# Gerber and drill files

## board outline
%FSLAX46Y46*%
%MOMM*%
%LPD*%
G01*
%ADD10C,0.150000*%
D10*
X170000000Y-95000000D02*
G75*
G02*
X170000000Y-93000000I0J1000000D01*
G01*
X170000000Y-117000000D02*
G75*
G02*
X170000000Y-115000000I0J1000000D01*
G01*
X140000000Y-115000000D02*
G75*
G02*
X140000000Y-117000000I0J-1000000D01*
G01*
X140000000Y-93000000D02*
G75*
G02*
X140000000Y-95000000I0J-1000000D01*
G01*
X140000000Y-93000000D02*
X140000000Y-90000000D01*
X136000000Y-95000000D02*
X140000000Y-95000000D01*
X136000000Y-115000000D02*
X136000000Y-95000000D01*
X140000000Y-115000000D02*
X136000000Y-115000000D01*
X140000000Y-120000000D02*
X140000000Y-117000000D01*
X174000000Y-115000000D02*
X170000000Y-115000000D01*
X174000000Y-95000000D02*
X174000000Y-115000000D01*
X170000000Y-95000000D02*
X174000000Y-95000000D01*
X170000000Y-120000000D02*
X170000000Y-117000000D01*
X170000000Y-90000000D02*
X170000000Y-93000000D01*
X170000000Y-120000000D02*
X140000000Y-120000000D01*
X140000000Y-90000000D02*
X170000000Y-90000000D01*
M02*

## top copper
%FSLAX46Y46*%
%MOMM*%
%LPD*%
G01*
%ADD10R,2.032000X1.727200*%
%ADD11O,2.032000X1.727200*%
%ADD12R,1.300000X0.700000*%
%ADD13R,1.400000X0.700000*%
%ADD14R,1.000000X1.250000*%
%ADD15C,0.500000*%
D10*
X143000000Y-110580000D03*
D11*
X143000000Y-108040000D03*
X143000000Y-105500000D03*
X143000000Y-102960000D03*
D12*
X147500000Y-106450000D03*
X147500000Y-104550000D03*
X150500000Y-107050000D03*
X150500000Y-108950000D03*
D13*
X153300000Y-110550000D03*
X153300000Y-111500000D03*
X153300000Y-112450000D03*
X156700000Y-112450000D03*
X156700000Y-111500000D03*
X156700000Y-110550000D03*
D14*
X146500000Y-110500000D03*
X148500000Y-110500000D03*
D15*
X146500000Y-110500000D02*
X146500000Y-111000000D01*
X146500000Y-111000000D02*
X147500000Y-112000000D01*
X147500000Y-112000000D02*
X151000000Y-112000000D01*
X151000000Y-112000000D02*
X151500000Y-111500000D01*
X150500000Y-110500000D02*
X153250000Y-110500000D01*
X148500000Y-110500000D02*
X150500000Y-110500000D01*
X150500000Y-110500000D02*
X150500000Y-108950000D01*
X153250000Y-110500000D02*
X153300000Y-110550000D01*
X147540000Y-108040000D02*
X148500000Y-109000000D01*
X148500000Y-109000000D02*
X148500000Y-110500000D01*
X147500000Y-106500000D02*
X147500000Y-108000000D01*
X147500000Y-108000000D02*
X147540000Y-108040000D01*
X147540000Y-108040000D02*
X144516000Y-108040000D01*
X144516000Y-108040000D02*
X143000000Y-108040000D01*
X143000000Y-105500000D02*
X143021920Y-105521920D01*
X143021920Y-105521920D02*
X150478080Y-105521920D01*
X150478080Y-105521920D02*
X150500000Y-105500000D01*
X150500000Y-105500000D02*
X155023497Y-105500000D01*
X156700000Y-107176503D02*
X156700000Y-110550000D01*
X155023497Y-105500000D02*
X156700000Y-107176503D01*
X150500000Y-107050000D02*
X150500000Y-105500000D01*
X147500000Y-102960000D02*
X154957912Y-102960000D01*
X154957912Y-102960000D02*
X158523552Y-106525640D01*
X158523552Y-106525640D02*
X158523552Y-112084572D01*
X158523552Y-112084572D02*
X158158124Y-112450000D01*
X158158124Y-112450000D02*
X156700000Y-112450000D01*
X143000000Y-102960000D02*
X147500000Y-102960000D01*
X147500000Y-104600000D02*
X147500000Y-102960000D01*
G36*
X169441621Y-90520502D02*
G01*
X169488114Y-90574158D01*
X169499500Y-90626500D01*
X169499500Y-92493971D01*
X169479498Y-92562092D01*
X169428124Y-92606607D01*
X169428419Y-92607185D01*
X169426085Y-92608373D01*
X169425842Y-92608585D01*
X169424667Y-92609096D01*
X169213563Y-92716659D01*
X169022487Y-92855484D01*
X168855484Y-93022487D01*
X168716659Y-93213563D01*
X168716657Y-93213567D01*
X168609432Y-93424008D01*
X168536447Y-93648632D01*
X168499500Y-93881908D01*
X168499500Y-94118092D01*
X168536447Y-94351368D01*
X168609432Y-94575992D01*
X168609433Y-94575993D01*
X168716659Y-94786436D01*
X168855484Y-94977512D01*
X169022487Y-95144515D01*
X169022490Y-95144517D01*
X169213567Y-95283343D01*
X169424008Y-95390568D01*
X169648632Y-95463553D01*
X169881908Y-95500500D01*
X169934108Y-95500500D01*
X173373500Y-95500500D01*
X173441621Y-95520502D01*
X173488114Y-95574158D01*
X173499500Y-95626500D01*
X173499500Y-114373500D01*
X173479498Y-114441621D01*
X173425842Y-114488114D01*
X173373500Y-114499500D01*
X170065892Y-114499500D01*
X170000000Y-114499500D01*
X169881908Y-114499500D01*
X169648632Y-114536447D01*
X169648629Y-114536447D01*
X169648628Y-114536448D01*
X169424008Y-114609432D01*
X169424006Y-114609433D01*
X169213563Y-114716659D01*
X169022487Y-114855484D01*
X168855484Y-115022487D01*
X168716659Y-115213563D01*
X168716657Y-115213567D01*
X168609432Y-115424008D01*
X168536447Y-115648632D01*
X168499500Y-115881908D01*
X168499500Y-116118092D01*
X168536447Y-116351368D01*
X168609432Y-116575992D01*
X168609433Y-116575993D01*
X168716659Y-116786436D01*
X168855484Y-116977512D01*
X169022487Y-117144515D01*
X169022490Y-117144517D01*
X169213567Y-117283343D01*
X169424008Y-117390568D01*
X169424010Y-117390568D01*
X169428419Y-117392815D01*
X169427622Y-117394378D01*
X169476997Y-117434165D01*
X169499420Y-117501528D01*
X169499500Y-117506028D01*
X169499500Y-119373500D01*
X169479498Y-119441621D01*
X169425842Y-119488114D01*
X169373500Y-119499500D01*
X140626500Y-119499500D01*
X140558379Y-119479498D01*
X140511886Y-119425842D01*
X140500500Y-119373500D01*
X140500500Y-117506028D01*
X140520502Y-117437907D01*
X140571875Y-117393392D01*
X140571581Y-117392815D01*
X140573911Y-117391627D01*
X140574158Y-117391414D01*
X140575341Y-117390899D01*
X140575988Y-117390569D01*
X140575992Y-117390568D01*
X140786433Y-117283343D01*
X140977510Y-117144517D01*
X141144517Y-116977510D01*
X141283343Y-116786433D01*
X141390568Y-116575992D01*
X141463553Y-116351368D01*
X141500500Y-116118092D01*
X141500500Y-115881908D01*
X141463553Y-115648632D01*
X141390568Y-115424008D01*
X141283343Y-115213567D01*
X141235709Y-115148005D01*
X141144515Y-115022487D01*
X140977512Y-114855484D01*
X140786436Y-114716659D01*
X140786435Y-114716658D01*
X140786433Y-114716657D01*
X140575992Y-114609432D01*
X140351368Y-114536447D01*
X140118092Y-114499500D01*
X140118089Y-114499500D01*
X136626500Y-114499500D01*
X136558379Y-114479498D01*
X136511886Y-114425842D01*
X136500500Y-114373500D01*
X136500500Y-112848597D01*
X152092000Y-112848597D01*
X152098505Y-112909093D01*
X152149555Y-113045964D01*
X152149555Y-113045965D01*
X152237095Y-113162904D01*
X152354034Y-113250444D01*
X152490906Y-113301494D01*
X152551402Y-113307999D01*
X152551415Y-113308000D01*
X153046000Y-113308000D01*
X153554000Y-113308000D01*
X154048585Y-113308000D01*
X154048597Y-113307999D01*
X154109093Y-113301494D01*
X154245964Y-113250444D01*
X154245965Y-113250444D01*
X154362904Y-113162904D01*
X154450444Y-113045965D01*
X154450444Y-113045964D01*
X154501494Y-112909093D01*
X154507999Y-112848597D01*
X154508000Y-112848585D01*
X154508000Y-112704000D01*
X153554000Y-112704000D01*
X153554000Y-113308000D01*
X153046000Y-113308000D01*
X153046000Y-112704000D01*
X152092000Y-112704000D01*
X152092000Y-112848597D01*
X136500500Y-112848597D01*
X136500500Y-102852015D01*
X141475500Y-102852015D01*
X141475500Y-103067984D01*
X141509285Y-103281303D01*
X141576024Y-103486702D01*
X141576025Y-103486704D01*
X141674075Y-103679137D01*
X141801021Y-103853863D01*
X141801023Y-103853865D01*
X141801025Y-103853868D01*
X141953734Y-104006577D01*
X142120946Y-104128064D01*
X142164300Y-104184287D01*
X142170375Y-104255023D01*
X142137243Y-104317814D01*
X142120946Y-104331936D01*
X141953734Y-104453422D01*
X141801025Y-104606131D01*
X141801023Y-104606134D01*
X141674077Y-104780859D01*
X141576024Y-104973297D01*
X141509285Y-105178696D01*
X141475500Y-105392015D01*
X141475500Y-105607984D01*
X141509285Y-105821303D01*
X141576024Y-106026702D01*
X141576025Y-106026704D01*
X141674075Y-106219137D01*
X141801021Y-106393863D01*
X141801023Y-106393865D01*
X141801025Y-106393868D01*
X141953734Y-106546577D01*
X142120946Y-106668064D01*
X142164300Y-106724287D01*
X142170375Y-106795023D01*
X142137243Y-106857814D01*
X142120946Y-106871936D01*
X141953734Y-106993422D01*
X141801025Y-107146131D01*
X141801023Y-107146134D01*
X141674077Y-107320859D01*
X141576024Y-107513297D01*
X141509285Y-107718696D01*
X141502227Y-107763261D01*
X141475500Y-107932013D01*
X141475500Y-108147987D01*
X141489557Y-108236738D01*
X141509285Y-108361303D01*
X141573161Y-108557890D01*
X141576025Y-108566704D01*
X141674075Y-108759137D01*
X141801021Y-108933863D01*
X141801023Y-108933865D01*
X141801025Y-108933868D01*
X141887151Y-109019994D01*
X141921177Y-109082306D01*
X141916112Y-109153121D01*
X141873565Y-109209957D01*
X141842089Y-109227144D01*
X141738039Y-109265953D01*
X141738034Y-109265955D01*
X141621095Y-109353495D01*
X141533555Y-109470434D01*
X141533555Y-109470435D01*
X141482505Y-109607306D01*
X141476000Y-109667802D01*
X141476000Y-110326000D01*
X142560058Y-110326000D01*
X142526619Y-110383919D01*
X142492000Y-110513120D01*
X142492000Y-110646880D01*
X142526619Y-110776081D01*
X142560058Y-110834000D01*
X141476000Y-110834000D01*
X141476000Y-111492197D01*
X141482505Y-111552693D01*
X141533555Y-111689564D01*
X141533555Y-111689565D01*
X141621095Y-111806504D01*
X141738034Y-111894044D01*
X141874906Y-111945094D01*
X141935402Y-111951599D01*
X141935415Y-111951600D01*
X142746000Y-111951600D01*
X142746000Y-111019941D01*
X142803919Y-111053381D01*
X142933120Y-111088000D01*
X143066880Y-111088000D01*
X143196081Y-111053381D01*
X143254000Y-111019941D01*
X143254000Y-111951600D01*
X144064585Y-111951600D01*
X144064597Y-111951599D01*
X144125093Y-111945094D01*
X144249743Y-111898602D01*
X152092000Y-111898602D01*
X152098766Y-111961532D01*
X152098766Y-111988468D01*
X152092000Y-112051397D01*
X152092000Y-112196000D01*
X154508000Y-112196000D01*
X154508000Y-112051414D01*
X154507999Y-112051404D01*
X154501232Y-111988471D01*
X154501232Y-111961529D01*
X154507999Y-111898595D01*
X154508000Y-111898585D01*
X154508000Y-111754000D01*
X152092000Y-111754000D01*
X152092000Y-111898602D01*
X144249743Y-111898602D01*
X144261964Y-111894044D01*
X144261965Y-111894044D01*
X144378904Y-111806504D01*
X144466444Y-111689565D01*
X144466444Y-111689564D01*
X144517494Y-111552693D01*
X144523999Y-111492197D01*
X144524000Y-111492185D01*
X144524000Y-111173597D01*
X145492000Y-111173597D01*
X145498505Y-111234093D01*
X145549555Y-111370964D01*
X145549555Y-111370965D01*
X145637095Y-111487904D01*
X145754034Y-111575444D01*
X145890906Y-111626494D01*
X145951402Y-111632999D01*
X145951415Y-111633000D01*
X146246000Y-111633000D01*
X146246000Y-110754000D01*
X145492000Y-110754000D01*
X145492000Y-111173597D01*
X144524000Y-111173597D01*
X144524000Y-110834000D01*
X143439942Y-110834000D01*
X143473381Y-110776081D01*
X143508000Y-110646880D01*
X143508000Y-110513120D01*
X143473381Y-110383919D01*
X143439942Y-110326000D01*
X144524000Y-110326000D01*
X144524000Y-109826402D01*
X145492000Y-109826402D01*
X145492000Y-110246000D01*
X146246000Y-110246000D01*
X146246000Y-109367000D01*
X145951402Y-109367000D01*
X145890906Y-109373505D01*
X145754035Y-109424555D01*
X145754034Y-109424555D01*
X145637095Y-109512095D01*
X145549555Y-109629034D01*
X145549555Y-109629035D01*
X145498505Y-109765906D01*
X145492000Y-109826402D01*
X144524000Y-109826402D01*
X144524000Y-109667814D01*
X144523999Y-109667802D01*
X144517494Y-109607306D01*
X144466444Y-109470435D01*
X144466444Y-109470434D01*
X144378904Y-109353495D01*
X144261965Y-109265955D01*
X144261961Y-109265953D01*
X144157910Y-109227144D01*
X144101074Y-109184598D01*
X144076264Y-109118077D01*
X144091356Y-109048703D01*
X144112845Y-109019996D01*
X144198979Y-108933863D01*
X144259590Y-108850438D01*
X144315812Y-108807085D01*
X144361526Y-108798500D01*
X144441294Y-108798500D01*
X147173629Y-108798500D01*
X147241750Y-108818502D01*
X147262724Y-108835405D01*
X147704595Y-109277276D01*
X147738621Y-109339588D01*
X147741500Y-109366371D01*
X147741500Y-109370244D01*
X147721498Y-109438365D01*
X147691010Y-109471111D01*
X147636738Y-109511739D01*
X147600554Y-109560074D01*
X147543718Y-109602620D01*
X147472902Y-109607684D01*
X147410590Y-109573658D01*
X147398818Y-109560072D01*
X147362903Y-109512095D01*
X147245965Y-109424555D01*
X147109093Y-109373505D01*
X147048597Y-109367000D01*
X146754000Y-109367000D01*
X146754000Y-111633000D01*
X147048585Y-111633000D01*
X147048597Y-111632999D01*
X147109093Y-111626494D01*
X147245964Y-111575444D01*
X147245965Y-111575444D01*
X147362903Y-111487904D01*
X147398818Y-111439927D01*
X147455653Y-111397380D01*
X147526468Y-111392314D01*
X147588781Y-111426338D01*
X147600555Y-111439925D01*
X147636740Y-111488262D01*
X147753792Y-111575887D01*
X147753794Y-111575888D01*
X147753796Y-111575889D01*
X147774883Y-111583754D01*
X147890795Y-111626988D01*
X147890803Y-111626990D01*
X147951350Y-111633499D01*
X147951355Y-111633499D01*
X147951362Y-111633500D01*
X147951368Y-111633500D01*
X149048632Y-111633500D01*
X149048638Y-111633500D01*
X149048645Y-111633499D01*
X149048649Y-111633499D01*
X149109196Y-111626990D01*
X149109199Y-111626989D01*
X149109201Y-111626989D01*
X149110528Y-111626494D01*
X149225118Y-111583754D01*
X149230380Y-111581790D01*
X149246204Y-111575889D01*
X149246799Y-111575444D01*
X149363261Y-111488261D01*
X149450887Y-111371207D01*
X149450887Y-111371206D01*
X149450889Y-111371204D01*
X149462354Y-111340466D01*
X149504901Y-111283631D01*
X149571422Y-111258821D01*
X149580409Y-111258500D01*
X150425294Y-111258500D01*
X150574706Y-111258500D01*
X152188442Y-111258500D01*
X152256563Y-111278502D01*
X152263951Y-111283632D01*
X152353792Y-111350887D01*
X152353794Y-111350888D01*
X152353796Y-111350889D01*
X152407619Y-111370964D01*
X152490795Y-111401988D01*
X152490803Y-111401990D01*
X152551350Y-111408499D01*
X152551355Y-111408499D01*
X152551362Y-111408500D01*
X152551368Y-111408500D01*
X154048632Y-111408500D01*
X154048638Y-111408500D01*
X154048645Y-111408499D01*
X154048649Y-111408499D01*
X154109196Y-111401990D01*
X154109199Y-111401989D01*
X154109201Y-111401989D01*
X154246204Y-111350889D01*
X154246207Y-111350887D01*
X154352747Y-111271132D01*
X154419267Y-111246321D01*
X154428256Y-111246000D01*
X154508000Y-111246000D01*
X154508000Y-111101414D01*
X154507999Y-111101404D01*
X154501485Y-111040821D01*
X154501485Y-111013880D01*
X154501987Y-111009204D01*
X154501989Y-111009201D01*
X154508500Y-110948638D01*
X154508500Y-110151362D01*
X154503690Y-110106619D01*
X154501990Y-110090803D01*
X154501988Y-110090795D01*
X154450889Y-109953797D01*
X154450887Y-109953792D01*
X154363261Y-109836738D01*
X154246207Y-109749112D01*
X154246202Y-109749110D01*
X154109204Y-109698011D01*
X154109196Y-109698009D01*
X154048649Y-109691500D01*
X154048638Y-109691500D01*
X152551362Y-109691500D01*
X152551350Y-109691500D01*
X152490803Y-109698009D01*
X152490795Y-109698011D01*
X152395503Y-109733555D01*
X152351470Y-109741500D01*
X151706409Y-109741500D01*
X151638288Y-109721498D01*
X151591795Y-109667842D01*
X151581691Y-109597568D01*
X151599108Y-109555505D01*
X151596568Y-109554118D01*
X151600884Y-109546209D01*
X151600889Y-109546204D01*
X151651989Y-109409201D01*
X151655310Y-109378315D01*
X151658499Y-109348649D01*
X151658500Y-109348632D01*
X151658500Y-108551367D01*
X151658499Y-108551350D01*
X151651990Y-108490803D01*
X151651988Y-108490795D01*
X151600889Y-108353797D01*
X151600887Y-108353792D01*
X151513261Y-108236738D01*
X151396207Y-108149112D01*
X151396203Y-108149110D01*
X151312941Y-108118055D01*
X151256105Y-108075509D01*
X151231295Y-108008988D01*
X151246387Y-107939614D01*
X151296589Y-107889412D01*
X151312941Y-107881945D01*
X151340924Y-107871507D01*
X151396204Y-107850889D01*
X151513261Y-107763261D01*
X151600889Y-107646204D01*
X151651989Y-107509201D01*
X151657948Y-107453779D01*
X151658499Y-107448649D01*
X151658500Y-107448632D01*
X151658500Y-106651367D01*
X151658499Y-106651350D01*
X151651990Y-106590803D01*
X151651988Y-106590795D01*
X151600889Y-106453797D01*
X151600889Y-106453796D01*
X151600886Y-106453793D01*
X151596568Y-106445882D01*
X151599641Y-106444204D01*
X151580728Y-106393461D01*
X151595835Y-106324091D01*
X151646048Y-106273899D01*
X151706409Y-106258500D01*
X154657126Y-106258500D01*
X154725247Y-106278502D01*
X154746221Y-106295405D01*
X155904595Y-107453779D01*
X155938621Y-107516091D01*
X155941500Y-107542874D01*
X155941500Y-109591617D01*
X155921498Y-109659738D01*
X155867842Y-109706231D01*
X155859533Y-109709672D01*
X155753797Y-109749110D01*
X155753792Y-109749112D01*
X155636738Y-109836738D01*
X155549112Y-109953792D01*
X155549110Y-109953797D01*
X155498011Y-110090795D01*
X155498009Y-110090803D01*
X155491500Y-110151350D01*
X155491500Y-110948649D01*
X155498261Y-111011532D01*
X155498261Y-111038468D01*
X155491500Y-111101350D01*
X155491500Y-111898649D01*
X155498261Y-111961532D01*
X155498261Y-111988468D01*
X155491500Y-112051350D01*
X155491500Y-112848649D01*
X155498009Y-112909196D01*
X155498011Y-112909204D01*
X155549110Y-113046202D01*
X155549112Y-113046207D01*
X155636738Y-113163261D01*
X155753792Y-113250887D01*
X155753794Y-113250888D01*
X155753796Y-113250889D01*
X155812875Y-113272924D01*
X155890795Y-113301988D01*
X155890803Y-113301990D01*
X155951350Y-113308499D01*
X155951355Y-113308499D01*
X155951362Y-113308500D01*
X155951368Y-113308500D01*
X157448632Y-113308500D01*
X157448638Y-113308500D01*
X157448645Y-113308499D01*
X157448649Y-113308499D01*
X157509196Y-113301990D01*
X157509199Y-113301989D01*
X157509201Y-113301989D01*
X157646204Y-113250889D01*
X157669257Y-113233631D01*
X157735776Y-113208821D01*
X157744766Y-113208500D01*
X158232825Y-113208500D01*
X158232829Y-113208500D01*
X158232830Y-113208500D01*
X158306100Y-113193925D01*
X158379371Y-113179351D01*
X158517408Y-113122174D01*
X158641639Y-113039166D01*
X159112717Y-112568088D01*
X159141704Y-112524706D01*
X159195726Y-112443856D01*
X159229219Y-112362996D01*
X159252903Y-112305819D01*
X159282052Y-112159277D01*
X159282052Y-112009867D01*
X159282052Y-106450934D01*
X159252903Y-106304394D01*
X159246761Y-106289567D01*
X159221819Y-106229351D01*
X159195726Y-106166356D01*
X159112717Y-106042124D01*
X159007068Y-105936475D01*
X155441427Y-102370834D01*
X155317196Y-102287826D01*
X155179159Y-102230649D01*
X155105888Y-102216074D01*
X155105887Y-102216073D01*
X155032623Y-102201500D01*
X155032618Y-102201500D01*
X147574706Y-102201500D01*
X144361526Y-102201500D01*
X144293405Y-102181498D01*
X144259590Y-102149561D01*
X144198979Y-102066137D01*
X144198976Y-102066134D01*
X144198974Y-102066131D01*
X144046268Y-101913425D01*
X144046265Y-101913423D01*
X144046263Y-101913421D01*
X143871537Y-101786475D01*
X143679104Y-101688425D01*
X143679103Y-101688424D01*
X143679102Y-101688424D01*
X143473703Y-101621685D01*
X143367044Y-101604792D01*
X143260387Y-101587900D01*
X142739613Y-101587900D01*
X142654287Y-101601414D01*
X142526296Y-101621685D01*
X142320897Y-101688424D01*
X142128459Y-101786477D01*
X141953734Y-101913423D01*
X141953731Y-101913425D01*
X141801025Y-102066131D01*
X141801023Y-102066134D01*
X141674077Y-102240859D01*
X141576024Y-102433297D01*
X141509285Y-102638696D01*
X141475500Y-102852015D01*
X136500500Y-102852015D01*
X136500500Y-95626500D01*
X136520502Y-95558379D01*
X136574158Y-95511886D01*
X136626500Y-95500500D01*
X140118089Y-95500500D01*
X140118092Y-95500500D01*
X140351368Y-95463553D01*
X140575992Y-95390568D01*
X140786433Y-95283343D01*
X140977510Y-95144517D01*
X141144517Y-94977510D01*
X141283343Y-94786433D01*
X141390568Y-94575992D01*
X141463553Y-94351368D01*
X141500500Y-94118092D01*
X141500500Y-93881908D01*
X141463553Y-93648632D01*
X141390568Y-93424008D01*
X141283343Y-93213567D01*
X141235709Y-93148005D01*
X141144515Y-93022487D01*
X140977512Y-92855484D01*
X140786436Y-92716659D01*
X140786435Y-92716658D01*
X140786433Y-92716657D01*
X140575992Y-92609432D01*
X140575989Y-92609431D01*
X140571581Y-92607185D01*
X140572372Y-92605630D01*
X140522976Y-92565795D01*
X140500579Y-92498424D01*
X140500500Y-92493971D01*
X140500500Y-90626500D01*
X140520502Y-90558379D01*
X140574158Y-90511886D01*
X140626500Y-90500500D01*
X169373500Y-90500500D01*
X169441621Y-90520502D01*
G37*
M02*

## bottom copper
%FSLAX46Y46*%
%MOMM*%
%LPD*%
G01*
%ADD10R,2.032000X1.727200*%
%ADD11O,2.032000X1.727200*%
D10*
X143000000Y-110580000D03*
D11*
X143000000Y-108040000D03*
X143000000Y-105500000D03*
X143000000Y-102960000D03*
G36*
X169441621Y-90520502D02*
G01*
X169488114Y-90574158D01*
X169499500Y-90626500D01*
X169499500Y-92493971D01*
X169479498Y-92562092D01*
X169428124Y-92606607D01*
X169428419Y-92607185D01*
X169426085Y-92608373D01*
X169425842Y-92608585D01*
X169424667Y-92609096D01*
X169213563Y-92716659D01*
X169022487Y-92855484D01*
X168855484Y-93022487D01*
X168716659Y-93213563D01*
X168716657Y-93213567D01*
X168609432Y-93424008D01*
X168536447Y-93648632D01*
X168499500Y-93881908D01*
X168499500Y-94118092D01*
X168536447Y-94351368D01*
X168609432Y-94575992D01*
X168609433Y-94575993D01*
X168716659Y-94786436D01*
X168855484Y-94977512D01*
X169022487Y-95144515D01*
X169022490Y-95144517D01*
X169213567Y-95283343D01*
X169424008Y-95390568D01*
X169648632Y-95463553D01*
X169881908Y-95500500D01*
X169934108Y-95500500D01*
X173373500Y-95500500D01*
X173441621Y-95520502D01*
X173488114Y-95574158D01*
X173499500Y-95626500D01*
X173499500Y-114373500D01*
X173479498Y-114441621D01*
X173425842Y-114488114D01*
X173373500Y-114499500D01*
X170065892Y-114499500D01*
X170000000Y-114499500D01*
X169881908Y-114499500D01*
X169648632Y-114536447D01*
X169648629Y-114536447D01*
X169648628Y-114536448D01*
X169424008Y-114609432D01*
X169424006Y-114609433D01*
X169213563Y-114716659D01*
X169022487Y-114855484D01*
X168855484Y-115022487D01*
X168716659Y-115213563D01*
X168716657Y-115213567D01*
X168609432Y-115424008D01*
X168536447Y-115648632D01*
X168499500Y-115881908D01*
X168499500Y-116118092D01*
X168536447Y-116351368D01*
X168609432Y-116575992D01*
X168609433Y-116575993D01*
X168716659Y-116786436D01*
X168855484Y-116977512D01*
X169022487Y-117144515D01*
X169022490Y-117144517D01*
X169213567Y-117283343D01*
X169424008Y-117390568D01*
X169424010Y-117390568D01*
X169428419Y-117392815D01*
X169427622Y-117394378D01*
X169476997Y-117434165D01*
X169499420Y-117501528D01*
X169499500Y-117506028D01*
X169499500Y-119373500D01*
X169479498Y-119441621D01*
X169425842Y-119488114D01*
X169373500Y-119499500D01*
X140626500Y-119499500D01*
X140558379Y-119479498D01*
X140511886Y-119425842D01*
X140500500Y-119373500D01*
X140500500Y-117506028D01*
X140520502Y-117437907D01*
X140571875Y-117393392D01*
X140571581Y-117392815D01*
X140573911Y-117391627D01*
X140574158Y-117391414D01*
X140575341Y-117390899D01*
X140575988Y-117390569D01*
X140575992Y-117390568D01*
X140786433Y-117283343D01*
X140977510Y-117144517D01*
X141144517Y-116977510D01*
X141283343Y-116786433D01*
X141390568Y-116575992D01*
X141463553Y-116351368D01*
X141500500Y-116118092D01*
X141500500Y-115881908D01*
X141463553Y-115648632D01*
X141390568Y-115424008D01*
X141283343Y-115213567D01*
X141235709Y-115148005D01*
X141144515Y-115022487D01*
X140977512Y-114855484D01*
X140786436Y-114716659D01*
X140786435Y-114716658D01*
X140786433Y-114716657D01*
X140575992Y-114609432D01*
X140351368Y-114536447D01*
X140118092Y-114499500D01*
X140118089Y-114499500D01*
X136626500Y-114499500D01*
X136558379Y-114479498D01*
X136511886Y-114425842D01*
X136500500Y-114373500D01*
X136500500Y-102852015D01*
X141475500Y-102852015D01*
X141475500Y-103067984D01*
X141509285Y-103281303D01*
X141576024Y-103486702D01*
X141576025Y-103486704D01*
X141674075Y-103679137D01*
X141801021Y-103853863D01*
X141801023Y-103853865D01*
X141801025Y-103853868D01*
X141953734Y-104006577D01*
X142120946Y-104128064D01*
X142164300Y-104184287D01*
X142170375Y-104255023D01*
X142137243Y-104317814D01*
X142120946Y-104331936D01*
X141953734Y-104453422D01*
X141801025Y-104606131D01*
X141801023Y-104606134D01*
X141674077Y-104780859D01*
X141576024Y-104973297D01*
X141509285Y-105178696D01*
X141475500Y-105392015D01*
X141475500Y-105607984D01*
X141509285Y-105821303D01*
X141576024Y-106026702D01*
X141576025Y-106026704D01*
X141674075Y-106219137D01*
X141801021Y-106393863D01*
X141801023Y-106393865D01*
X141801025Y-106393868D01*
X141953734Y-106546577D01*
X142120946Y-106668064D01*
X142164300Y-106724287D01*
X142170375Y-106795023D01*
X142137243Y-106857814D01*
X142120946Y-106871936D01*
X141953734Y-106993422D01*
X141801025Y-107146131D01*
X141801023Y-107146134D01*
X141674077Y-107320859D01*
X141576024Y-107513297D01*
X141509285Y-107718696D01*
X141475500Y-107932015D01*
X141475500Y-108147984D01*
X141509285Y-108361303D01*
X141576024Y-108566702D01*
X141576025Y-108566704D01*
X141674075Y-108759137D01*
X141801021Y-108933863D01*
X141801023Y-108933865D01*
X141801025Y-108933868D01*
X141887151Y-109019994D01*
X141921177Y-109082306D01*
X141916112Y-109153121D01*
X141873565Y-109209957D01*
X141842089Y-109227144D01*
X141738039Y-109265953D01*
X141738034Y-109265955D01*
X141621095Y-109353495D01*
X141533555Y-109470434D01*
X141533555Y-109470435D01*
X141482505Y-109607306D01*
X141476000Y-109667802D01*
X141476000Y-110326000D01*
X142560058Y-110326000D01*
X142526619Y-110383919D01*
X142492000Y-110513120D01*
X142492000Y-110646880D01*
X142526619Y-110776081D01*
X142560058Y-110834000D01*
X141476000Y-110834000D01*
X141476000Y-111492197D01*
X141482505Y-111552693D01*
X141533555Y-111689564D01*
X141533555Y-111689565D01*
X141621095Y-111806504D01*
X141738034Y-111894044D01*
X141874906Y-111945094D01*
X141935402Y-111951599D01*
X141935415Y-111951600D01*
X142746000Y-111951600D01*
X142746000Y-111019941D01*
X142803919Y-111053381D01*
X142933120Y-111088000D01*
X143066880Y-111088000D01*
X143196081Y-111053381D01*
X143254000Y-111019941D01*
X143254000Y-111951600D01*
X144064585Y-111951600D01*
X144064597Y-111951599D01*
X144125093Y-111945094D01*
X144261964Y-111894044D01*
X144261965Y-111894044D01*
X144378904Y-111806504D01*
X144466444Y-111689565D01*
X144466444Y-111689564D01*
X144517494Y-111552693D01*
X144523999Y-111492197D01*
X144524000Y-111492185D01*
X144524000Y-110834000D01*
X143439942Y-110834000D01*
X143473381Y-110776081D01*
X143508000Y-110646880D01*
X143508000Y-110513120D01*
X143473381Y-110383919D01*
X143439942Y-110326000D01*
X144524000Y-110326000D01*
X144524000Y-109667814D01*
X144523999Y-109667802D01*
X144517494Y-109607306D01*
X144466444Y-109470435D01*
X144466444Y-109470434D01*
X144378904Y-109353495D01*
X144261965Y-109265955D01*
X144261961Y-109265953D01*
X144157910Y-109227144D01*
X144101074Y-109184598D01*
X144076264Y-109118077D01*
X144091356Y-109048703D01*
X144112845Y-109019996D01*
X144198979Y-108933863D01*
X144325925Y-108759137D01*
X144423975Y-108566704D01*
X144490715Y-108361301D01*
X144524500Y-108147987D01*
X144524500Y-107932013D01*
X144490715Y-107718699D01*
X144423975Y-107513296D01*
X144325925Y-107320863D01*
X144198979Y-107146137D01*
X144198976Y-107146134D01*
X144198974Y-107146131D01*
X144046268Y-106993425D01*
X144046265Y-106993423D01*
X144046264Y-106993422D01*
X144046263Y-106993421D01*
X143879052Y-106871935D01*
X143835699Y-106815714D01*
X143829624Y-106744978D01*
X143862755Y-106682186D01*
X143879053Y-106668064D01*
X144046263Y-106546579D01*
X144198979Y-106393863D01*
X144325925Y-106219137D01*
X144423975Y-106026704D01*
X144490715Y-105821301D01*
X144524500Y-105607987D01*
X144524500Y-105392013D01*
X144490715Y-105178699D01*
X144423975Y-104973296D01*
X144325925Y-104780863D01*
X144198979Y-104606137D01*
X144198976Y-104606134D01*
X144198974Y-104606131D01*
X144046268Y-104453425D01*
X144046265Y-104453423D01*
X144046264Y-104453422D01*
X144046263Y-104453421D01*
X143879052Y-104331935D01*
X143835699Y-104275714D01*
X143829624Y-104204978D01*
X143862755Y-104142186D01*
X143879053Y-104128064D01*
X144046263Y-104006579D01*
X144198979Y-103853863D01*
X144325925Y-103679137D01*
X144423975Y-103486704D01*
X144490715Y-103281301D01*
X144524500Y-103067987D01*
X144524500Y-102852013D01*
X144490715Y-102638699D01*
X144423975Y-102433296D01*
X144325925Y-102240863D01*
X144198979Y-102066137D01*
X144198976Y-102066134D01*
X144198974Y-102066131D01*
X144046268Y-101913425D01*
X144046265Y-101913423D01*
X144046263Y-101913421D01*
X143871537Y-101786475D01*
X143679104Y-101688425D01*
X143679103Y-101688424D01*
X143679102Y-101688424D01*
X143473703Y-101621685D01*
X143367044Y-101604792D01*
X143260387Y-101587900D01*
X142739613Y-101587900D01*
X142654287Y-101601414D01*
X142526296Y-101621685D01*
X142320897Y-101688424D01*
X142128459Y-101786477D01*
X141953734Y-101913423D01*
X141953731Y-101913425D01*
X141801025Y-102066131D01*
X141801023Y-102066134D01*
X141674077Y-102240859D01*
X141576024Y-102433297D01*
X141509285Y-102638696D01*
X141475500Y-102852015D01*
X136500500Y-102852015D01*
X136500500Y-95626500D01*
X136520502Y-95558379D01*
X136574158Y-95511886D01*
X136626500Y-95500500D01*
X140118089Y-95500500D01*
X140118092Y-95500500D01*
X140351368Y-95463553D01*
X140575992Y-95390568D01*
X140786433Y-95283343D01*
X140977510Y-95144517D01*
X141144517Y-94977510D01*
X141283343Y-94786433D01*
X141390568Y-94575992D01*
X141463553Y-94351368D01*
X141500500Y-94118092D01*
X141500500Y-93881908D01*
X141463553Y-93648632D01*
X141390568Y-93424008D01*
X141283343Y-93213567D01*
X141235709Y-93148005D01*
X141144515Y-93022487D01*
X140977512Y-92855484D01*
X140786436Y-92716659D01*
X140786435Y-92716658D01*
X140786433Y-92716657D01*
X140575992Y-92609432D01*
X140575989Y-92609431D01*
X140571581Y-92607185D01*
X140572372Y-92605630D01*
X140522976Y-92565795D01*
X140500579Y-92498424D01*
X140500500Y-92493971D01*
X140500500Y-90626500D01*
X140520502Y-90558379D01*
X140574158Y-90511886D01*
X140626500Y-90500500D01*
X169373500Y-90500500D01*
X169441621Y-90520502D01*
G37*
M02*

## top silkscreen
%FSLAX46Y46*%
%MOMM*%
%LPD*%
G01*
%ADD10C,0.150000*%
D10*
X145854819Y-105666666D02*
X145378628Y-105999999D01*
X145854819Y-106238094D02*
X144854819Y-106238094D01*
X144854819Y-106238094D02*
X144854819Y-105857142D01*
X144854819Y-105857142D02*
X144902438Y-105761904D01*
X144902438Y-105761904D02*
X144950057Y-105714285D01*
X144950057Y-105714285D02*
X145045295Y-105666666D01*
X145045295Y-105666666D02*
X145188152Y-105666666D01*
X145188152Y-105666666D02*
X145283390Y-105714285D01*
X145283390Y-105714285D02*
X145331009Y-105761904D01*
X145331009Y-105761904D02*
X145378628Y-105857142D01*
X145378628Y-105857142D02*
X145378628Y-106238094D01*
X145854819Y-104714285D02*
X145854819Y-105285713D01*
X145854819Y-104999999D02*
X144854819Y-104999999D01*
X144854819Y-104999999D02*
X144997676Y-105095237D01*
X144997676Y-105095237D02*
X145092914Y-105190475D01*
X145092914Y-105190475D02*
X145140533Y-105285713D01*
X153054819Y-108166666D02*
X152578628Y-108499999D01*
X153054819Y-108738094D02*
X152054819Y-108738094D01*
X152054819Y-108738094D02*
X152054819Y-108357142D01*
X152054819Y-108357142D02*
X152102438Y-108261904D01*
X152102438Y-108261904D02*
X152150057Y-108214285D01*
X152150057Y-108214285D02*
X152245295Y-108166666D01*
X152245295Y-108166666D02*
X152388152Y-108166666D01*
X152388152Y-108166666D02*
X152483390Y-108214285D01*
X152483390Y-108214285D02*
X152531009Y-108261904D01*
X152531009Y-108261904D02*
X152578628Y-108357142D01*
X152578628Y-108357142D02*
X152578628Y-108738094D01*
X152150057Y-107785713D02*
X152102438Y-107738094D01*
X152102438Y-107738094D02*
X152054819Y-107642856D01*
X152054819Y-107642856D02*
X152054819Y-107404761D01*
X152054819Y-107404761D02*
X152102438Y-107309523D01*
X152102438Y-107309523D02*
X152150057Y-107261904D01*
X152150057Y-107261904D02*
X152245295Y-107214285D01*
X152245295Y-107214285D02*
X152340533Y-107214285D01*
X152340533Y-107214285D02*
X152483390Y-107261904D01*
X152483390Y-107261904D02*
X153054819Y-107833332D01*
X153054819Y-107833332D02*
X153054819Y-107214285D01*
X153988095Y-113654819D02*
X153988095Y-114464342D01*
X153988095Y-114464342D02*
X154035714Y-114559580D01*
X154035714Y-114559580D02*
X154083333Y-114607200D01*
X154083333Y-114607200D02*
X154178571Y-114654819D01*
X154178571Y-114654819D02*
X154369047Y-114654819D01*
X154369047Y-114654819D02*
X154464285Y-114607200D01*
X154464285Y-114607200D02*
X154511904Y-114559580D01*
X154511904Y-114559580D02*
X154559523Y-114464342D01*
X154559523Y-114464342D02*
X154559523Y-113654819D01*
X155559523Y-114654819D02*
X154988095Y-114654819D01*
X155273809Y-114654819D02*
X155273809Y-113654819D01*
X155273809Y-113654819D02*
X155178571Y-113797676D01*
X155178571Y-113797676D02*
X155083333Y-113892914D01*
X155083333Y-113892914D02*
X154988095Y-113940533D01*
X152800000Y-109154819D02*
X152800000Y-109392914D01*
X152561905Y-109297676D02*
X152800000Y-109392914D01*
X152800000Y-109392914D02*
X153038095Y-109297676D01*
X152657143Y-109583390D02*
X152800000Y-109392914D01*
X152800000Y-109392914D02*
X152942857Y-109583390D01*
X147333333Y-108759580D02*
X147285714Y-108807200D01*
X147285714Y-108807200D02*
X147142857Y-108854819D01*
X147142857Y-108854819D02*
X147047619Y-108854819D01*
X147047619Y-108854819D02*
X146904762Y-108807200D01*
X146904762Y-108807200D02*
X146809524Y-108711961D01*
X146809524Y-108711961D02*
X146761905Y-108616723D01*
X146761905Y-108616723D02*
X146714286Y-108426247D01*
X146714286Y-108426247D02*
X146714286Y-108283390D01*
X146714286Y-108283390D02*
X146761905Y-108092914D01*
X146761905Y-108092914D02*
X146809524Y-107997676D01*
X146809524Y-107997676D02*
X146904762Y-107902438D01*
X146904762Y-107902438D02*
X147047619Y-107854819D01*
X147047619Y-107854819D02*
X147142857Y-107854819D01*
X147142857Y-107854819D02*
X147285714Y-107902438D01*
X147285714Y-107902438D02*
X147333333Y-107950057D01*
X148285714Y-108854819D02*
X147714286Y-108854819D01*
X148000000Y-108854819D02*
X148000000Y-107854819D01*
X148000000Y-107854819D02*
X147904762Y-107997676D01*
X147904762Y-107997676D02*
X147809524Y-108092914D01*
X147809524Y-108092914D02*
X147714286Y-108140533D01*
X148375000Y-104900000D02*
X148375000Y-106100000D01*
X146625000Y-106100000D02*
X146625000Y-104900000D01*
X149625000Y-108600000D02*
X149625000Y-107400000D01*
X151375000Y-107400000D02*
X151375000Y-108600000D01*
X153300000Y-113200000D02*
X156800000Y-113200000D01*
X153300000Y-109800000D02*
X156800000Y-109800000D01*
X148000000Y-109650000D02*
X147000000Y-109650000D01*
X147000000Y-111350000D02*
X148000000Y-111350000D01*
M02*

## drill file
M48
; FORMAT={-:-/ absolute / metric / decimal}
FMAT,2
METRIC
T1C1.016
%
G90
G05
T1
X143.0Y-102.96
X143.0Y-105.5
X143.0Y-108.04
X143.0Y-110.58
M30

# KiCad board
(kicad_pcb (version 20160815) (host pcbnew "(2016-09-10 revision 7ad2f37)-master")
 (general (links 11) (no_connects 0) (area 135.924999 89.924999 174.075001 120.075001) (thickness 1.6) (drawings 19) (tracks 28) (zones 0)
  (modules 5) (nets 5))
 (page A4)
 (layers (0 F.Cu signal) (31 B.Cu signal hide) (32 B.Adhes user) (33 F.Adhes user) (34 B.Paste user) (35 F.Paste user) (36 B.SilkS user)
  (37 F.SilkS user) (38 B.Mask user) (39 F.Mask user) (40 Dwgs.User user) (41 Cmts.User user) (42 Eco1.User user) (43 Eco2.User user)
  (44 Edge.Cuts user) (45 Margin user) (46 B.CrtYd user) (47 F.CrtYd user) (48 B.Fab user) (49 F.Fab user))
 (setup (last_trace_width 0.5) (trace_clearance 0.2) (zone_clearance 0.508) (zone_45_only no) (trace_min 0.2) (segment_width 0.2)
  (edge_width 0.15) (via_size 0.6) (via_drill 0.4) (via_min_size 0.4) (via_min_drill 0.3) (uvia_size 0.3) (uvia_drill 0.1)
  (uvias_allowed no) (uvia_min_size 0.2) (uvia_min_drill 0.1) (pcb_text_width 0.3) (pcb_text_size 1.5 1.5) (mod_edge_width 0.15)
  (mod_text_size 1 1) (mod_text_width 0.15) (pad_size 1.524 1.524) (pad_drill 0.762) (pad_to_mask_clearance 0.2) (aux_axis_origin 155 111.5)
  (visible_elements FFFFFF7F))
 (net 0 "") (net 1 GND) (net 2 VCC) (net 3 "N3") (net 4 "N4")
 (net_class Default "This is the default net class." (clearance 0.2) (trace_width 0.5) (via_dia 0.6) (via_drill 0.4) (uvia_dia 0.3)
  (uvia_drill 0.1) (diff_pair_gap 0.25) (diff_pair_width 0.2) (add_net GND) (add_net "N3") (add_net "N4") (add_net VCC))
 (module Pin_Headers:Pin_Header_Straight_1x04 (layer B.Cu) (at 143 110.58)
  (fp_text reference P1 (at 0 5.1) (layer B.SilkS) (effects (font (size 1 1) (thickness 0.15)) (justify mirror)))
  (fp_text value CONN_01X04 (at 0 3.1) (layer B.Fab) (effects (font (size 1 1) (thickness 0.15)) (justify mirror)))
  (pad 1 thru_hole rect (at 0 0) (size 2.032 1.7272) (drill 1.016) (layers *.Cu *.Mask B.SilkS) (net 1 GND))
  (pad 2 thru_hole oval (at 0 -2.54) (size 2.032 1.7272) (drill 1.016) (layers *.Cu *.Mask B.SilkS) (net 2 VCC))
  (pad 3 thru_hole oval (at 0 -5.08) (size 2.032 1.7272) (drill 1.016) (layers *.Cu *.Mask B.SilkS) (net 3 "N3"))
  (pad 4 thru_hole oval (at 0 -7.62) (size 2.032 1.7272) (drill 1.016) (layers *.Cu *.Mask B.SilkS) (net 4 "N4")))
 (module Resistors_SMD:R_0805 (layer F.Cu) (at 147.5 105.5 90)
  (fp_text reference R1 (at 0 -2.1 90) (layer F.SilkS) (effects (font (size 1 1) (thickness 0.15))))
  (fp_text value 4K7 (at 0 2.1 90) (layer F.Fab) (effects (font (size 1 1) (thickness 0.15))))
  (fp_line (start 0.6 0.875) (end -0.6 0.875) (layer F.SilkS) (width 0.15))
  (fp_line (start -0.6 -0.875) (end 0.6 -0.875) (layer F.SilkS) (width 0.15))
  (pad 1 smd rect (at -0.95 0 90) (size 0.7 1.3) (layers F.Cu F.Paste F.Mask) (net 2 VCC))
  (pad 2 smd rect (at 0.95 0 90) (size 0.7 1.3) (layers F.Cu F.Paste F.Mask) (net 4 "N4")))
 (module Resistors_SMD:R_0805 (layer F.Cu) (at 150.5 108 270)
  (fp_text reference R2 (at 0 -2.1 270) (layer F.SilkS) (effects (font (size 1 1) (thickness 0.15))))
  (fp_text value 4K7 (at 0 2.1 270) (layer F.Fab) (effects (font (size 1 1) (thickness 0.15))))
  (fp_line (start 0.6 0.875) (end -0.6 0.875) (layer F.SilkS) (width 0.15))
  (fp_line (start -0.6 -0.875) (end 0.6 -0.875) (layer F.SilkS) (width 0.15))
  (pad 1 smd rect (at -0.95 0 270) (size 0.7 1.3) (layers F.Cu F.Paste F.Mask) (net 3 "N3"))
  (pad 2 smd rect (at 0.95 0 270) (size 0.7 1.3) (layers F.Cu F.Paste F.Mask) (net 2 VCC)))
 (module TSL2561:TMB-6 (layer F.Cu) (at 155 111.5)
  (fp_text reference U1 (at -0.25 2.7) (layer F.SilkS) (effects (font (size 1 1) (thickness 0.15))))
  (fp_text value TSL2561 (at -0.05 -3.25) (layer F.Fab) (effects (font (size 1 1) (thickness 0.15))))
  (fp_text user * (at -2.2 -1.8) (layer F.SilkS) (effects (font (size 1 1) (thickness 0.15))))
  (fp_line (start -1.7 1.7) (end 1.8 1.7) (layer F.SilkS) (width 0.15))
  (fp_line (start -1.7 -1.7) (end 1.8 -1.7) (layer F.SilkS) (width 0.15))
  (pad 1 smd rect (at -1.7 -0.95) (size 1.4 0.7) (layers F.Cu F.Paste F.Mask) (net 2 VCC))
  (pad 2 smd rect (at -1.7 0) (size 1.4 0.7) (layers F.Cu F.Paste F.Mask) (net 1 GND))
  (pad 3 smd rect (at -1.7 0.95) (size 1.4 0.7) (layers F.Cu F.Paste F.Mask) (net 1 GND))
  (pad 4 smd rect (at 1.7 0.95) (size 1.4 0.7) (layers F.Cu F.Paste F.Mask) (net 4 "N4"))
  (pad 5 smd rect (at 1.7 0) (size 1.4 0.7) (layers F.Cu F.Paste F.Mask))
  (pad 6 smd rect (at 1.7 -0.95) (size 1.4 0.7) (layers F.Cu F.Paste F.Mask) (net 3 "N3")))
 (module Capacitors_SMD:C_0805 (layer F.Cu) (at 147.5 110.5)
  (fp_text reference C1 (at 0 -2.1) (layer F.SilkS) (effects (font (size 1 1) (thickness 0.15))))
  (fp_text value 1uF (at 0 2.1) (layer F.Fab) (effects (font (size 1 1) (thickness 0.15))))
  (fp_line (start 0.5 -0.85) (end -0.5 -0.85) (layer F.SilkS) (width 0.15))
  (fp_line (start -0.5 0.85) (end 0.5 0.85) (layer F.SilkS) (width 0.15))
  (pad 1 smd rect (at -1 0) (size 1 1.25) (layers F.Cu F.Paste F.Mask) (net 1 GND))
  (pad 2 smd rect (at 1 0) (size 1 1.25) (layers F.Cu F.Paste F.Mask) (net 2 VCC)))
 (gr_arc (start 170 94) (end 170 95) (angle 180) (layer Edge.Cuts) (width 0.15))
 (gr_arc (start 170 116) (end 170 117) (angle 180) (layer Edge.Cuts) (width 0.15))
 (gr_arc (start 140 116) (end 140 115) (angle 180) (layer Edge.Cuts) (width 0.15))
 (gr_arc (start 140 94) (end 140 93) (angle 180) (layer Edge.Cuts) (width 0.15))
 (gr_line (start 140 93) (end 140 90) (layer Edge.Cuts) (width 0.15))
 (gr_line (start 136 95) (end 140 95) (layer Edge.Cuts) (width 0.15))
 (gr_line (start 136 115) (end 136 95) (layer Edge.Cuts) (width 0.15))
 (gr_line (start 140 115) (end 136 115) (layer Edge.Cuts) (width 0.15))
 (gr_line (start 140 120) (end 140 117) (layer Edge.Cuts) (width 0.15))
 (gr_line (start 174 115) (end 170 115) (layer Edge.Cuts) (width 0.15))
 (gr_line (start 174 95) (end 174 115) (layer Edge.Cuts) (width 0.15))
 (gr_line (start 170 95) (end 174 95) (layer Edge.Cuts) (width 0.15))
 (gr_line (start 170 120) (end 170 117) (layer Edge.Cuts) (width 0.15))
 (gr_line (start 170 90) (end 170 93) (layer Edge.Cuts) (width 0.15))
 (gr_line (start 170 120) (end 140 120) (layer Edge.Cuts) (width 0.15))
 (gr_line (start 140 90) (end 170 90) (layer Edge.Cuts) (width 0.15))
 (segment (start 146.5 110.5) (end 146.5 111) (width 0.5) (layer F.Cu) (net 1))
 (segment (start 146.5 111) (end 147.5 112) (width 0.5) (layer F.Cu) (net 1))
 (segment (start 147.5 112) (end 151 112) (width 0.5) (layer F.Cu) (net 1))
 (segment (start 151 112) (end 151.5 111.5) (width 0.5) (layer F.Cu) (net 1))
 (segment (start 150.5 110.5) (end 153.25 110.5) (width 0.5) (layer F.Cu) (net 2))
 (segment (start 148.5 110.5) (end 150.5 110.5) (width 0.5) (layer F.Cu) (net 2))
 (segment (start 150.5 110.5) (end 150.5 108.95) (width 0.5) (layer F.Cu) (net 2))
 (segment (start 153.25 110.5) (end 153.3 110.55) (width 0.5) (layer F.Cu) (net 2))
 (segment (start 147.54 108.04) (end 148.5 109) (width 0.5) (layer F.Cu) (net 2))
 (segment (start 148.5 109) (end 148.5 110.5) (width 0.5) (layer F.Cu) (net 2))
 (segment (start 147.5 106.5) (end 147.5 108) (width 0.5) (layer F.Cu) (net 2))
 (segment (start 147.5 108) (end 147.54 108.04) (width 0.5) (layer F.Cu) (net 2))
 (segment (start 147.54 108.04) (end 144.516 108.04) (width 0.5) (layer F.Cu) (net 2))
 (segment (start 144.516 108.04) (end 143 108.04) (width 0.5) (layer F.Cu) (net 2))
 (segment (start 143 105.5) (end 143.02192 105.52192) (width 0.5) (layer F.Cu) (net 3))
 (segment (start 143.02192 105.52192) (end 150.47808 105.52192) (width 0.5) (layer F.Cu) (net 3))
 (segment (start 150.47808 105.52192) (end 150.5 105.5) (width 0.5) (layer F.Cu) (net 3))
 (segment (start 150.5 105.5) (end 155.023497 105.5) (width 0.5) (layer F.Cu) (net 3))
 (segment (start 156.7 107.176503) (end 156.7 110.55) (width 0.5) (layer F.Cu) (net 3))
 (segment (start 155.023497 105.5) (end 156.7 107.176503) (width 0.5) (layer F.Cu) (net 3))
 (segment (start 150.5 107.05) (end 150.5 105.5) (width 0.5) (layer F.Cu) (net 3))
 (segment (start 147.5 102.96) (end 154.957912 102.96) (width 0.5) (layer F.Cu) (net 4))
 (segment (start 154.957912 102.96) (end 158.523552 106.52564) (width 0.5) (layer F.Cu) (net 4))
 (segment (start 158.523552 106.52564) (end 158.523552 112.084572) (width 0.5) (layer F.Cu) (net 4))
 (segment (start 158.523552 112.084572) (end 158.158124 112.45) (width 0.5) (layer F.Cu) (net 4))
 (segment (start 158.158124 112.45) (end 156.7 112.45) (width 0.5) (layer F.Cu) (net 4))
 (segment (start 143 102.96) (end 147.5 102.96) (width 0.5) (layer F.Cu) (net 4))
 (segment (start 147.5 104.6) (end 147.5 102.96) (width 0.5) (layer F.Cu) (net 4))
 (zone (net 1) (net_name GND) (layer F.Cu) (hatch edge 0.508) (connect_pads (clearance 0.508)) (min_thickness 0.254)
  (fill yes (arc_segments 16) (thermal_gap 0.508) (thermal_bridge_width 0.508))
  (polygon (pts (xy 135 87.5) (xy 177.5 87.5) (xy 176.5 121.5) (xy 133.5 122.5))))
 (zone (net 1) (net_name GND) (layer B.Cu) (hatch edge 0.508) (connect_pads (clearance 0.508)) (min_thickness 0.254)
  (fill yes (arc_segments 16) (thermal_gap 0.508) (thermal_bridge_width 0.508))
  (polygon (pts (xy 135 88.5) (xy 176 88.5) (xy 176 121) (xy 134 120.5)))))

